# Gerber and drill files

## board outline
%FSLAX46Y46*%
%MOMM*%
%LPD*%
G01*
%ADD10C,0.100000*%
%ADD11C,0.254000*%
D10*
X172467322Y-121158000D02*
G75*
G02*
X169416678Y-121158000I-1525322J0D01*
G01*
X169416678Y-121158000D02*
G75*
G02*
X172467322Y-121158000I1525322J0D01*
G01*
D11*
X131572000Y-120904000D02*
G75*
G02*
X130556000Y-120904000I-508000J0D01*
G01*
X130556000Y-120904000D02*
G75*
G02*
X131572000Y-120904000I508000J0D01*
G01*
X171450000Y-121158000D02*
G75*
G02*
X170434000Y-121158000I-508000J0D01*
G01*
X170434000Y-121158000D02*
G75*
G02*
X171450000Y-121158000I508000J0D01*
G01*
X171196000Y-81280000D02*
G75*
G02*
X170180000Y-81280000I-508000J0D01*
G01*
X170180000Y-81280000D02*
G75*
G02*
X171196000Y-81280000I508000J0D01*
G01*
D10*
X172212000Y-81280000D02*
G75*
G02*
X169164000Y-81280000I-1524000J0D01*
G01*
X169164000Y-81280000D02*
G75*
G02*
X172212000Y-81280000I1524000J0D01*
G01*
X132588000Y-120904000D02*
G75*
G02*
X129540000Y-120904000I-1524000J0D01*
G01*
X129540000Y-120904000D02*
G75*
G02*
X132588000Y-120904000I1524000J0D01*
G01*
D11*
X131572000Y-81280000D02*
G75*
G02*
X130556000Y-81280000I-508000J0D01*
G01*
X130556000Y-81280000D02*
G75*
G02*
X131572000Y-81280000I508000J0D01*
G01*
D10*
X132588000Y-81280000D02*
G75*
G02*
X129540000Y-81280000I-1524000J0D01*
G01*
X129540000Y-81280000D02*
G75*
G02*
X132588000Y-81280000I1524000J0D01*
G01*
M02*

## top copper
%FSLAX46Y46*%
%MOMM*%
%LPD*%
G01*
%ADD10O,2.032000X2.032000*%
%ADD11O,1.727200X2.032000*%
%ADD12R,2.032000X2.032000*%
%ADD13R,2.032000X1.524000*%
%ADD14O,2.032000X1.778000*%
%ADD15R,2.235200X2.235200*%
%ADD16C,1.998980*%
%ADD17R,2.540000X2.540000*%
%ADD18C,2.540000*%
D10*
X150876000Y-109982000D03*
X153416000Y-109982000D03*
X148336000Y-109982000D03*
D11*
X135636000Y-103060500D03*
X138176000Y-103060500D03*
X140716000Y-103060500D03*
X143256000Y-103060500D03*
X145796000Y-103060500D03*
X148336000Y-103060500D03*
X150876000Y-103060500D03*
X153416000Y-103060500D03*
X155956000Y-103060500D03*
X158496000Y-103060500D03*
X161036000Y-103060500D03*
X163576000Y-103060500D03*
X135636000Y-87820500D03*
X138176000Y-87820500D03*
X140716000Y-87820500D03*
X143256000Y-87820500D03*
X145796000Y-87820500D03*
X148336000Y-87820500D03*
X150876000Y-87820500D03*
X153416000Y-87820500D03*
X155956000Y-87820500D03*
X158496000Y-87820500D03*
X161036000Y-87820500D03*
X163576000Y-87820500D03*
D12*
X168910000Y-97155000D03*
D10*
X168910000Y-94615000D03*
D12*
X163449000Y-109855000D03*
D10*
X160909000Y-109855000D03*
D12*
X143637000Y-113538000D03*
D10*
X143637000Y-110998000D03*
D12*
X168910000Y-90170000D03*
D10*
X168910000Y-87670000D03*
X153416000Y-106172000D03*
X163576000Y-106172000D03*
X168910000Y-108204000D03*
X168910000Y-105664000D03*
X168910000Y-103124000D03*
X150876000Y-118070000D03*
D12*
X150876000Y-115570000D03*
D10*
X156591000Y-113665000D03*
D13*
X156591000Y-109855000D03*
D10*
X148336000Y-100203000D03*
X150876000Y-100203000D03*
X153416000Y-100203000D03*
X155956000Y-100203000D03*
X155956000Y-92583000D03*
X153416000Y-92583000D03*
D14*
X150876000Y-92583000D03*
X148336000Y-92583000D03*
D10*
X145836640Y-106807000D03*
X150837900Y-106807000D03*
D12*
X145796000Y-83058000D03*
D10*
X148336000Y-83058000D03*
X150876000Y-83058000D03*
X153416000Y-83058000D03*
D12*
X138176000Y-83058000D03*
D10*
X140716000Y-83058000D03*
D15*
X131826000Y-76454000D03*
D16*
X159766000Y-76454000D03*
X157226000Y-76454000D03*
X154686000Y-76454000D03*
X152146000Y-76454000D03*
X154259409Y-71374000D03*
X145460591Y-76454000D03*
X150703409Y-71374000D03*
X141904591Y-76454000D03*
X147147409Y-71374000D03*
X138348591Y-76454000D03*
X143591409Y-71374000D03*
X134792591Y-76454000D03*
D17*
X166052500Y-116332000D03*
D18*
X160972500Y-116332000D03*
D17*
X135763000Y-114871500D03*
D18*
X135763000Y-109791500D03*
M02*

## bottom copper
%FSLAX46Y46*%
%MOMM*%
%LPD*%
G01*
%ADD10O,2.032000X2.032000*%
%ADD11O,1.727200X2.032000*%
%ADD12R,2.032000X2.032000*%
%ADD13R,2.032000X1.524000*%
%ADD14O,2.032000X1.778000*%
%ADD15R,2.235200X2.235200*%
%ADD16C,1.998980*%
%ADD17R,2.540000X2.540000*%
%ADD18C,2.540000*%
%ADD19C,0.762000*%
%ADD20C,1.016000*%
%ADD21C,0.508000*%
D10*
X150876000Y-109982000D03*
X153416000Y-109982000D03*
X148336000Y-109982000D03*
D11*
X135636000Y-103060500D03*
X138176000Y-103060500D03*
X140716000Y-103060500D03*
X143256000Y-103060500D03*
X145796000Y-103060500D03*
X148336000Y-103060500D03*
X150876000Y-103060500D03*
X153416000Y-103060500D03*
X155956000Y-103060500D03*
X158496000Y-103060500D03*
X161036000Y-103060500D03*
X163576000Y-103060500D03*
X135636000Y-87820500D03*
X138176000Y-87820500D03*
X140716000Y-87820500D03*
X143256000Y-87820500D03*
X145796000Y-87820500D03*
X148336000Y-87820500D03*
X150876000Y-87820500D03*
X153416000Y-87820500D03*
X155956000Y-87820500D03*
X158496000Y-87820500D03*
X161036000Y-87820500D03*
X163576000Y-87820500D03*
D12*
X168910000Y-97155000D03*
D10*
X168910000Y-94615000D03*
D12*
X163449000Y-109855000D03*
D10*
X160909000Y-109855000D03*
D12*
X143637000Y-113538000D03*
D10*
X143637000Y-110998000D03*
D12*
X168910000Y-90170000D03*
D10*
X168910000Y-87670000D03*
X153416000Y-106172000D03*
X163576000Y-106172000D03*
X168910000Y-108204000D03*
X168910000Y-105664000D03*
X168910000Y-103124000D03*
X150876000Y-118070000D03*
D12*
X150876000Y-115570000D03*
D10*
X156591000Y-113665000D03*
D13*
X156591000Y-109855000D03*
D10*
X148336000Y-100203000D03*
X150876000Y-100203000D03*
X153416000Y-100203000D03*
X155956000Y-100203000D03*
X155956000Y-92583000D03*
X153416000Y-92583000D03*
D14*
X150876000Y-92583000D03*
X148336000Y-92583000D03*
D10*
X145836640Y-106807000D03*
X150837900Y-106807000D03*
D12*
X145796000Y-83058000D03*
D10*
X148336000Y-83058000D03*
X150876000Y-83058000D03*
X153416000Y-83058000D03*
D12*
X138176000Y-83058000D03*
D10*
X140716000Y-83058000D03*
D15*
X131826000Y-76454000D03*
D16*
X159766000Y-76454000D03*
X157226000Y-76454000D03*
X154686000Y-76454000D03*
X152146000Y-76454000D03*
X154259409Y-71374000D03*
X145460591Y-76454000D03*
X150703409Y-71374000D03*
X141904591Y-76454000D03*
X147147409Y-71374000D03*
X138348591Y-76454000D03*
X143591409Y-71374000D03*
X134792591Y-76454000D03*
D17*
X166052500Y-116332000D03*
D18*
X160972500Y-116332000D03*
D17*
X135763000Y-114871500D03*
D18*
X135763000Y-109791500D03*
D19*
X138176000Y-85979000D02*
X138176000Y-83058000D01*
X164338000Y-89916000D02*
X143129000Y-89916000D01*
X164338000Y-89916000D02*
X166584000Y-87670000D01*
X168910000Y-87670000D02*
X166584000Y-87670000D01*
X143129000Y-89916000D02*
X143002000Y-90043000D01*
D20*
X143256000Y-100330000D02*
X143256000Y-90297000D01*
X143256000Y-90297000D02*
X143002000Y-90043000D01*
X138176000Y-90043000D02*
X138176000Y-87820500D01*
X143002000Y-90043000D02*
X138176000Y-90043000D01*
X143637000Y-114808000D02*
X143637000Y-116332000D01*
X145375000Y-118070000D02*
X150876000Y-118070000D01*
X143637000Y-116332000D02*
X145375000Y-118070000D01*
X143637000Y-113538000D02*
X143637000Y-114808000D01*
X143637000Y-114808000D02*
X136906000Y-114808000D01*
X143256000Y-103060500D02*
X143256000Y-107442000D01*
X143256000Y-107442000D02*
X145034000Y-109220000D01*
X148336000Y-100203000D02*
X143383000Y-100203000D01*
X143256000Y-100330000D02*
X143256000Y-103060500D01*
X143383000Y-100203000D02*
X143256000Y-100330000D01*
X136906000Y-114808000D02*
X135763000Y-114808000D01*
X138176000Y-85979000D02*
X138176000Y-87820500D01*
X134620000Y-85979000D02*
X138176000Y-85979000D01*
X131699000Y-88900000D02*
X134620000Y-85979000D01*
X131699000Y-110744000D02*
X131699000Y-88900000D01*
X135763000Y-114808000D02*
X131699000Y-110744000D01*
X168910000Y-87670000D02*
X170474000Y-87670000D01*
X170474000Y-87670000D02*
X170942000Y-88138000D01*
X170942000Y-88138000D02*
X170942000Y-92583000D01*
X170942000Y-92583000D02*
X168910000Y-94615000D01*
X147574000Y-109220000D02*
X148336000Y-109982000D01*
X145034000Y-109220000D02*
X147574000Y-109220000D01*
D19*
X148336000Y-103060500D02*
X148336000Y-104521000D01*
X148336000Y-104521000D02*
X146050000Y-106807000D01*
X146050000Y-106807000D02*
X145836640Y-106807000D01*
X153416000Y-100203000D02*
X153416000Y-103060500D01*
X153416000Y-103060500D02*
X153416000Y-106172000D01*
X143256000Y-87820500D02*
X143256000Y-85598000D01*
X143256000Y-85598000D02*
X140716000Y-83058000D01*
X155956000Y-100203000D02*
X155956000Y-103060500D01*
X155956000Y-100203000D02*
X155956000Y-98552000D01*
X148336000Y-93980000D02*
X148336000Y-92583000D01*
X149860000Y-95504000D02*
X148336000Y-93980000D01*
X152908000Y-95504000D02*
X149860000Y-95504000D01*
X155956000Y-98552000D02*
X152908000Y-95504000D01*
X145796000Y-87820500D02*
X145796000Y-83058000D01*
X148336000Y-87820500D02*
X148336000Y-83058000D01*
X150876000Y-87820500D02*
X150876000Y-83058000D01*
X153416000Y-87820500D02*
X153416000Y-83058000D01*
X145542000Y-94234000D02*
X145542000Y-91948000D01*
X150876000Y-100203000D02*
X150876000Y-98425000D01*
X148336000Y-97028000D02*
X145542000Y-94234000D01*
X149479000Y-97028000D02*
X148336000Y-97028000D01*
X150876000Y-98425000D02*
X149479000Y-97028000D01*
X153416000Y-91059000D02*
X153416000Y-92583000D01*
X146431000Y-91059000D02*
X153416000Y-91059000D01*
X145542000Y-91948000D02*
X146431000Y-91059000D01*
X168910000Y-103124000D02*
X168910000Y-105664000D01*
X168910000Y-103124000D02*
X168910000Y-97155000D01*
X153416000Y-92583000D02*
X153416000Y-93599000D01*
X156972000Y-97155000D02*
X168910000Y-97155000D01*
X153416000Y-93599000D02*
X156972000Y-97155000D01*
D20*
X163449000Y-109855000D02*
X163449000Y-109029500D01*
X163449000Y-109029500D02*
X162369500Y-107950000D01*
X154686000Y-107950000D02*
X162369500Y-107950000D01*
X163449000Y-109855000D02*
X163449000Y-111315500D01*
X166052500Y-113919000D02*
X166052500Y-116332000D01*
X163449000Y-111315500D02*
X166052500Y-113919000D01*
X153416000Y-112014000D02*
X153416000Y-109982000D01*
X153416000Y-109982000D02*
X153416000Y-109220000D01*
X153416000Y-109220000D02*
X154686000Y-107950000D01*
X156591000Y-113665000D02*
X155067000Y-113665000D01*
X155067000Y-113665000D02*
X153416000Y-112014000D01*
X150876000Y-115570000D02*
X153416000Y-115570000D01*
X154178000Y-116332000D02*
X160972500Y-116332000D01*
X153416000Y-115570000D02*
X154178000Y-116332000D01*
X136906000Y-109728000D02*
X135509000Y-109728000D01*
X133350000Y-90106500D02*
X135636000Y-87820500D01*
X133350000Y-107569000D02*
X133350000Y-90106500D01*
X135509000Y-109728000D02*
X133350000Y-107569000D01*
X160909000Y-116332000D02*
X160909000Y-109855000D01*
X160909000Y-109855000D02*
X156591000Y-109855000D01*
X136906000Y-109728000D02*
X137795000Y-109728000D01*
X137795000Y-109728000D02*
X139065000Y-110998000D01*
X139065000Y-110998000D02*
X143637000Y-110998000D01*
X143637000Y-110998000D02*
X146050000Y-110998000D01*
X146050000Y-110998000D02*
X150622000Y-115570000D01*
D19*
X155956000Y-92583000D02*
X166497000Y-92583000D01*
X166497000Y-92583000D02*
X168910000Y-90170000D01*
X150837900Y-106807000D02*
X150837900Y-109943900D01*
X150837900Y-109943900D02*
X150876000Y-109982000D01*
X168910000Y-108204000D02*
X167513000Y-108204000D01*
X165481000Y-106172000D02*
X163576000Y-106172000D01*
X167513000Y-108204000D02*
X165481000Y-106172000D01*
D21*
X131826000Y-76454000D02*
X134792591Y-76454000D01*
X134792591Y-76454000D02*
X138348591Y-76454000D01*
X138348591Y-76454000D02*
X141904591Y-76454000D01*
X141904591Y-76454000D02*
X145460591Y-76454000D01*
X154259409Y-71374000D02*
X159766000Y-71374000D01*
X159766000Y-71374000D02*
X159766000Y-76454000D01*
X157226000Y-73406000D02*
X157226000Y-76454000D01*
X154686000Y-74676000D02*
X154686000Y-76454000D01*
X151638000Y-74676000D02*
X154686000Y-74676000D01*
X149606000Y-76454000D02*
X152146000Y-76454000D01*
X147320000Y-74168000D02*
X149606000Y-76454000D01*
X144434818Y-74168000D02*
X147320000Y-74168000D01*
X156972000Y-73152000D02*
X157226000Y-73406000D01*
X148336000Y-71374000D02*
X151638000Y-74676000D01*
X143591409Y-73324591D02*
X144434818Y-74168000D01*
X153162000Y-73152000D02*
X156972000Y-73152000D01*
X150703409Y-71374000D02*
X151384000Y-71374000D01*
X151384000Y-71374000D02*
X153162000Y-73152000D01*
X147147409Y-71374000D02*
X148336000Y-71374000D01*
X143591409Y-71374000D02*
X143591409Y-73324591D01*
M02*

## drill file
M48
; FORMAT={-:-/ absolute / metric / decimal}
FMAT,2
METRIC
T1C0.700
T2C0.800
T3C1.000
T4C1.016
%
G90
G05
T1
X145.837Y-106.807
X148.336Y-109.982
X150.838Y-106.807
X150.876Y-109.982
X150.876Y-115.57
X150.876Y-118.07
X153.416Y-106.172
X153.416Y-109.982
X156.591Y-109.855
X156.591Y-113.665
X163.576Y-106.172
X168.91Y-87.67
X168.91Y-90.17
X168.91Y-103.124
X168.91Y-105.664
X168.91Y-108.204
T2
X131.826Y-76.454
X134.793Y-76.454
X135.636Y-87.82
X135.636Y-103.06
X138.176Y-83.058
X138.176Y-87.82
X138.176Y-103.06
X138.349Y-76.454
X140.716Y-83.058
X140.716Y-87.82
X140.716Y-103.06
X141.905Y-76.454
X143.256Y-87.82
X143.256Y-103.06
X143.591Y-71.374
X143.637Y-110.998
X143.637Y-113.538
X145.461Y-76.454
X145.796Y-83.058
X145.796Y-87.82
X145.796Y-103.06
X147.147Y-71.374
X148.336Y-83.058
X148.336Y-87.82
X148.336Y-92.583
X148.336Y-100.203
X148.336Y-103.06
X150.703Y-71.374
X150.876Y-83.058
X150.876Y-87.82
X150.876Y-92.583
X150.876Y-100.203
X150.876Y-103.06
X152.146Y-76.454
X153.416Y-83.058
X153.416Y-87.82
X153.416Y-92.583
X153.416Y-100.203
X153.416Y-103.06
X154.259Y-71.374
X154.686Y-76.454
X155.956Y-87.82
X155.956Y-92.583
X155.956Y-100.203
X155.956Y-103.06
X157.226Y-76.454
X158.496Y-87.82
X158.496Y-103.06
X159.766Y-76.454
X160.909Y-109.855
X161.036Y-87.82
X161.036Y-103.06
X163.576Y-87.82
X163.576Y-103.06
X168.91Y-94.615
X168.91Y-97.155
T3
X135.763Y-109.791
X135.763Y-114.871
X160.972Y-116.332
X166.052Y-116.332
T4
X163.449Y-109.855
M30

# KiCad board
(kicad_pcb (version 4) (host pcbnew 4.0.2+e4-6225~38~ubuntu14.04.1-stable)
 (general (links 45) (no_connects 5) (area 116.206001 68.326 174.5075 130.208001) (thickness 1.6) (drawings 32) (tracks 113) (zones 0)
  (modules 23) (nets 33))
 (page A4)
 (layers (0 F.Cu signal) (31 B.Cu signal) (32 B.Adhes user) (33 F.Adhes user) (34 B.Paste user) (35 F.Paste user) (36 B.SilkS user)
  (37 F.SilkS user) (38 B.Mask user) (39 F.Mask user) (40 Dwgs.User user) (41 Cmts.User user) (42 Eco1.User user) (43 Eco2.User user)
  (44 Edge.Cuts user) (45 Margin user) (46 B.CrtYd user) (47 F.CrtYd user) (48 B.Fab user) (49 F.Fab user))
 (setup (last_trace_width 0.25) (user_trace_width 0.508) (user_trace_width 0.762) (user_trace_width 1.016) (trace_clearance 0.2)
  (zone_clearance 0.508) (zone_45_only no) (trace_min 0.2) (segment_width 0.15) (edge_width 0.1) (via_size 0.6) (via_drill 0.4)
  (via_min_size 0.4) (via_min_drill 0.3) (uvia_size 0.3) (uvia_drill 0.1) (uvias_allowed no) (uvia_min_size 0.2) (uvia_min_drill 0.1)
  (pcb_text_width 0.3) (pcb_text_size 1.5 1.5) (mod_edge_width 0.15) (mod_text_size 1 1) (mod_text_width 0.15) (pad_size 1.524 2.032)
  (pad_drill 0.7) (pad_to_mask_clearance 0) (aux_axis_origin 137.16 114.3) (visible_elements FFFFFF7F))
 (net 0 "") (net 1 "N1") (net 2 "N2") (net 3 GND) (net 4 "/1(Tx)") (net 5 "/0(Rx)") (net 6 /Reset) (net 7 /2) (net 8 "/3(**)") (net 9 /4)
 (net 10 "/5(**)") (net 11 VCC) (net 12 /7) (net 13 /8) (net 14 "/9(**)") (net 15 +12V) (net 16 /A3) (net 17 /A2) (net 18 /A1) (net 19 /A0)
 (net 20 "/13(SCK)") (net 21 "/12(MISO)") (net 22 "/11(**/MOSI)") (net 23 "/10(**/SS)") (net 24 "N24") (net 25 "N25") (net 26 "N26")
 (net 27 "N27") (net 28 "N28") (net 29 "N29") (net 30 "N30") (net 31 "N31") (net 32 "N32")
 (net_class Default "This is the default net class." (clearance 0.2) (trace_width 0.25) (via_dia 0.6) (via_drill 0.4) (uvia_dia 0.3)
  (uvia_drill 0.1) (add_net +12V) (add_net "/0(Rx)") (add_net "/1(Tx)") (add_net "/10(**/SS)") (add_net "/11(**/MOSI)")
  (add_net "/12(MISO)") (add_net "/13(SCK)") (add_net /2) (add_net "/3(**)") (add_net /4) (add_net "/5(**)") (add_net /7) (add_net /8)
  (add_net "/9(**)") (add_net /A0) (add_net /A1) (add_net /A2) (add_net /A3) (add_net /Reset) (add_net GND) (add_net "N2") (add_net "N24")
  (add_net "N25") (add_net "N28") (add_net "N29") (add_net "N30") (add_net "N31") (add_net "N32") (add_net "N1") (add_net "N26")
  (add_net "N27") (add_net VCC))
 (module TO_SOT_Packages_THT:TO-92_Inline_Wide (layer F.Cu) (at 148.336 109.982)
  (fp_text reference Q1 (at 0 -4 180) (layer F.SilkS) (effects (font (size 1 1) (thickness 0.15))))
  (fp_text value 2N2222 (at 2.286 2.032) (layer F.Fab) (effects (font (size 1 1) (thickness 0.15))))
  (pad 2 thru_hole oval (at 2.54 0) (size 2.032 2.032) (drill 0.7) (layers *.Cu *.Mask F.SilkS) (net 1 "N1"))
  (pad 3 thru_hole oval (at 5.08 0) (size 2.032 2.032) (drill 0.7) (layers *.Cu *.Mask F.SilkS) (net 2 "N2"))
  (pad 1 thru_hole oval (at 0 0) (size 2.032 2.032) (drill 0.7) (layers *.Cu *.Mask F.SilkS) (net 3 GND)))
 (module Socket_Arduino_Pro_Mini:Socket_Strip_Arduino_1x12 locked (layer F.Cu) (at 135.636 103.0605)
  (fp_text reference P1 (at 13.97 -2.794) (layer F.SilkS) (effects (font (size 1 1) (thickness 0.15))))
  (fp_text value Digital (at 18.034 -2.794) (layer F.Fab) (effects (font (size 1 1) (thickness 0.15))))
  (pad 1 thru_hole oval (at 0 0) (size 1.7272 2.032) (drill 0.8) (layers *.Cu *.Mask F.SilkS) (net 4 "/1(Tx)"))
  (pad 2 thru_hole oval (at 2.54 0) (size 1.7272 2.032) (drill 0.8) (layers *.Cu *.Mask F.SilkS) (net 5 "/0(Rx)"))
  (pad 3 thru_hole oval (at 5.08 0) (size 1.7272 2.032) (drill 0.8) (layers *.Cu *.Mask F.SilkS) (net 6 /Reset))
  (pad 4 thru_hole oval (at 7.62 0) (size 1.7272 2.032) (drill 0.8) (layers *.Cu *.Mask F.SilkS) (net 3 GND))
  (pad 5 thru_hole oval (at 10.16 0) (size 1.7272 2.032) (drill 0.8) (layers *.Cu *.Mask F.SilkS) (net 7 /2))
  (pad 6 thru_hole oval (at 12.7 0) (size 1.7272 2.032) (drill 0.8) (layers *.Cu *.Mask F.SilkS) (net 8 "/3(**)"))
  (pad 7 thru_hole oval (at 15.24 0) (size 1.7272 2.032) (drill 0.8) (layers *.Cu *.Mask F.SilkS) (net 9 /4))
  (pad 8 thru_hole oval (at 17.78 0) (size 1.7272 2.032) (drill 0.8) (layers *.Cu *.Mask F.SilkS) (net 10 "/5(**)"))
  (pad 9 thru_hole oval (at 20.32 0) (size 1.7272 2.032) (drill 0.8) (layers *.Cu *.Mask F.SilkS) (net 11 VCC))
  (pad 10 thru_hole oval (at 22.86 0) (size 1.7272 2.032) (drill 0.8) (layers *.Cu *.Mask F.SilkS) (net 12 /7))
  (pad 11 thru_hole oval (at 25.4 0) (size 1.7272 2.032) (drill 0.8) (layers *.Cu *.Mask F.SilkS) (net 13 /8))
  (pad 12 thru_hole oval (at 27.94 0) (size 1.7272 2.032) (drill 0.8) (layers *.Cu *.Mask F.SilkS) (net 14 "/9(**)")))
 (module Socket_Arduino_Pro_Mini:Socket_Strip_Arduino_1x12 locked (layer F.Cu) (at 135.636 87.8205)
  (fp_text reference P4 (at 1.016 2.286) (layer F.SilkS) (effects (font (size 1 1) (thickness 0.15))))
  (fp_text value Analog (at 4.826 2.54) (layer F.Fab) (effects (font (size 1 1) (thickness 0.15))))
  (pad 1 thru_hole oval (at 0 0) (size 1.7272 2.032) (drill 0.8) (layers *.Cu *.Mask F.SilkS) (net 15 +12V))
  (pad 2 thru_hole oval (at 2.54 0) (size 1.7272 2.032) (drill 0.8) (layers *.Cu *.Mask F.SilkS) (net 3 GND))
  (pad 3 thru_hole oval (at 5.08 0) (size 1.7272 2.032) (drill 0.8) (layers *.Cu *.Mask F.SilkS) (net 6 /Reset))
  (pad 4 thru_hole oval (at 7.62 0) (size 1.7272 2.032) (drill 0.8) (layers *.Cu *.Mask F.SilkS) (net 11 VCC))
  (pad 5 thru_hole oval (at 10.16 0) (size 1.7272 2.032) (drill 0.8) (layers *.Cu *.Mask F.SilkS) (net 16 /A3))
  (pad 6 thru_hole oval (at 12.7 0) (size 1.7272 2.032) (drill 0.8) (layers *.Cu *.Mask F.SilkS) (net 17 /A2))
  (pad 7 thru_hole oval (at 15.24 0) (size 1.7272 2.032) (drill 0.8) (layers *.Cu *.Mask F.SilkS) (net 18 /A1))
  (pad 8 thru_hole oval (at 17.78 0) (size 1.7272 2.032) (drill 0.8) (layers *.Cu *.Mask F.SilkS) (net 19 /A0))
  (pad 9 thru_hole oval (at 20.32 0) (size 1.7272 2.032) (drill 0.8) (layers *.Cu *.Mask F.SilkS) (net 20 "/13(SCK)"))
  (pad 10 thru_hole oval (at 22.86 0) (size 1.7272 2.032) (drill 0.8) (layers *.Cu *.Mask F.SilkS) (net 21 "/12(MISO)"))
  (pad 11 thru_hole oval (at 25.4 0) (size 1.7272 2.032) (drill 0.8) (layers *.Cu *.Mask F.SilkS) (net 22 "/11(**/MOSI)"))
  (pad 12 thru_hole oval (at 27.94 0) (size 1.7272 2.032) (drill 0.8) (layers *.Cu *.Mask F.SilkS) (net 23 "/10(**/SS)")))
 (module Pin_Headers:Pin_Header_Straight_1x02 (layer F.Cu) (at 168.91 97.155 180)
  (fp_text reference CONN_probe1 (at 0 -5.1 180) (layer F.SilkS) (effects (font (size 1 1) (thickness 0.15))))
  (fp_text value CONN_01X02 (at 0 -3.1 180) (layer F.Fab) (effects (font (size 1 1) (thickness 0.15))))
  (pad 1 thru_hole rect (at 0 0 180) (size 2.032 2.032) (drill 0.8) (layers *.Cu *.Mask F.SilkS) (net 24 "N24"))
  (pad 2 thru_hole oval (at 0 2.54 180) (size 2.032 2.032) (drill 0.8) (layers *.Cu *.Mask F.SilkS) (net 3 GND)))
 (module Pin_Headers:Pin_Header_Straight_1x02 (layer F.Cu) (at 163.449 109.855 270)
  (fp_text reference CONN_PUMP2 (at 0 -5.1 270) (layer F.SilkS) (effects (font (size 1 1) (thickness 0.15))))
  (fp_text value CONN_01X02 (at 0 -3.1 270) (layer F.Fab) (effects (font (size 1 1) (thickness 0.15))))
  (pad 1 thru_hole rect (at 0 0 270) (size 2.032 2.032) (drill 1.016) (layers *.Cu *.Mask F.SilkS) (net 2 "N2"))
  (pad 2 thru_hole oval (at 0 2.54 270) (size 2.032 2.032) (drill 0.8) (layers *.Cu *.Mask F.SilkS) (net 15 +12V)))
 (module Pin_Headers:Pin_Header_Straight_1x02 (layer F.Cu) (at 143.637 113.538 180)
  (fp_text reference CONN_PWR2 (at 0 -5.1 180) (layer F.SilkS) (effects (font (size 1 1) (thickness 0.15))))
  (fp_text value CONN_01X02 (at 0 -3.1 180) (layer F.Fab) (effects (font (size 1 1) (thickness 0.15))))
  (pad 1 thru_hole rect (at 0 0 180) (size 2.032 2.032) (drill 0.8) (layers *.Cu *.Mask F.SilkS) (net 3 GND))
  (pad 2 thru_hole oval (at 0 2.54 180) (size 2.032 2.032) (drill 0.8) (layers *.Cu *.Mask F.SilkS) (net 15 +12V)))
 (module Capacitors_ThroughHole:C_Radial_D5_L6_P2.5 (layer F.Cu) (at 168.91 90.17 90)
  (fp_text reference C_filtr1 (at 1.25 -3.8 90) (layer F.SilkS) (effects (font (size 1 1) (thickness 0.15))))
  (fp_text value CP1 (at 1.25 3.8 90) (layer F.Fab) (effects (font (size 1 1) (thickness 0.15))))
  (pad 1 thru_hole rect (at 0 0 90) (size 2.032 2.032) (drill 0.7) (layers *.Cu *.Mask F.SilkS) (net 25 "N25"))
  (pad 2 thru_hole oval (at 2.5 0 90) (size 2.032 2.032) (drill 0.7) (layers *.Cu *.Mask F.SilkS) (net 3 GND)))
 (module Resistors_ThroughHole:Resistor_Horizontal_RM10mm (layer F.Cu) (at 158.496 106.172)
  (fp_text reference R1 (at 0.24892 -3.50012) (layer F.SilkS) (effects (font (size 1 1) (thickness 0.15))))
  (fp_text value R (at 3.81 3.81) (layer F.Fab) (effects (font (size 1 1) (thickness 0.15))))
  (pad 1 thru_hole oval (at -5.08 0) (size 2.032 2.032) (drill 0.7) (layers *.Cu *.Mask F.SilkS) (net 10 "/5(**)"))
  (pad 2 thru_hole oval (at 5.08 0) (size 2.032 2.032) (drill 0.7) (layers *.Cu *.Mask F.SilkS) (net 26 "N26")))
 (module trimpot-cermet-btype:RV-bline (layer F.Cu) (at 168.91 105.664 90)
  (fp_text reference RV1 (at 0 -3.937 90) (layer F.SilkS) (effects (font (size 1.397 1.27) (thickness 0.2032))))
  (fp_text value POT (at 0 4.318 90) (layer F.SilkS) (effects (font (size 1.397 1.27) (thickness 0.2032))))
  (pad 1 thru_hole oval (at -2.54 0 90) (size 2.032 2.032) (drill 0.7) (layers *.Cu *.Mask F.SilkS) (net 26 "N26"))
  (pad 2 thru_hole oval (at 0 0 90) (size 2.032 2.032) (drill 0.7) (layers *.Cu *.Mask F.SilkS) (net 24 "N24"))
  (pad 3 thru_hole oval (at 2.54 0 90) (size 2.032 2.032) (drill 0.7) (layers *.Cu *.Mask F.SilkS) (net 24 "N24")))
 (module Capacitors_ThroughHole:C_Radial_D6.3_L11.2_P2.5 (layer F.Cu) (at 150.876 115.57 270)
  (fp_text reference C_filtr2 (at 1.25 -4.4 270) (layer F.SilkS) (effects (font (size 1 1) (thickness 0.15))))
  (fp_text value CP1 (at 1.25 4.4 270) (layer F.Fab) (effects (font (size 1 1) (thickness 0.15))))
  (pad 2 thru_hole oval (at 2.5 0 270) (size 2.032 2.032) (drill 0.7) (layers *.Cu *.Mask F.SilkS) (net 3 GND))
  (pad 1 thru_hole rect (at 0 0 270) (size 2.032 2.032) (drill 0.7) (layers *.Cu *.Mask F.SilkS) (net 15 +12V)))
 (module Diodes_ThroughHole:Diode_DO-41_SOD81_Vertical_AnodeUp (layer F.Cu) (at 156.591 109.855 270)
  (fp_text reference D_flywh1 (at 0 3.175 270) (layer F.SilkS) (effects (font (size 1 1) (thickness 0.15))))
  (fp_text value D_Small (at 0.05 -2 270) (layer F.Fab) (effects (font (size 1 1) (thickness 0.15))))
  (pad 2 thru_hole oval (at 3.81 0 270) (size 2.032 2.032) (drill 0.7) (layers *.Cu *.Mask F.SilkS) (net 2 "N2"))
  (pad 1 thru_hole rect (at 0 0 270) (size 1.524 2.032) (drill 0.7) (layers *.Cu *.Mask F.SilkS) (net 15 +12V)))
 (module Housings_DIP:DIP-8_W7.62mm (layer F.Cu) (at 148.336 100.203 90)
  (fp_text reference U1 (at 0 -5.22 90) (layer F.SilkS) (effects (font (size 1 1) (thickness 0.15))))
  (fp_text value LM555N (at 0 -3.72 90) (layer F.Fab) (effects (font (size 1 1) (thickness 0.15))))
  (pad 1 thru_hole oval (at 0 0 90) (size 2.032 2.032) (drill 0.8) (layers *.Cu *.Mask F.SilkS) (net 3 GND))
  (pad 2 thru_hole oval (at 0 2.54 90) (size 2.032 2.032) (drill 0.8) (layers *.Cu *.Mask F.SilkS) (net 24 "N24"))
  (pad 3 thru_hole oval (at 0 5.08 90) (size 2.032 2.032) (drill 0.8) (layers *.Cu *.Mask F.SilkS) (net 10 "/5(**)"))
  (pad 4 thru_hole oval (at 0 7.62 90) (size 2.032 2.032) (drill 0.8) (layers *.Cu *.Mask F.SilkS) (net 11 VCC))
  (pad 5 thru_hole oval (at 7.62 7.62 90) (size 2.032 2.032) (drill 0.8) (layers *.Cu *.Mask F.SilkS) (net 25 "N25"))
  (pad 6 thru_hole oval (at 7.62 5.08 90) (size 2.032 2.032) (drill 0.8) (layers *.Cu *.Mask F.SilkS) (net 24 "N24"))
  (pad 7 thru_hole oval (at 7.62 2.54 90) (size 1.778 2.032) (drill 0.8) (layers *.Cu *.Mask F.SilkS) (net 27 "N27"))
  (pad 8 thru_hole oval (at 7.62 0 90) (size 1.778 2.032) (drill 0.8) (layers *.Cu *.Mask F.SilkS) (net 11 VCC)))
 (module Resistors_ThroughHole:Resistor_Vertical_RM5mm (layer F.Cu) (at 148.336 106.807)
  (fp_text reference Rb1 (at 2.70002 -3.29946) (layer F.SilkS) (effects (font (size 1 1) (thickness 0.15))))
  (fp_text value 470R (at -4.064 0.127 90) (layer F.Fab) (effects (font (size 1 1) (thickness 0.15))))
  (pad 1 thru_hole oval (at -2.49936 0) (size 2.032 2.032) (drill 0.7) (layers *.Cu *.Mask F.SilkS) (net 8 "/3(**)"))
  (pad 2 thru_hole oval (at 2.5019 0) (size 2.032 2.032) (drill 0.7) (layers *.Cu *.Mask F.SilkS) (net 1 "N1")))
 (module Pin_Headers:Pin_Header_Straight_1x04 (layer F.Cu) (at 145.796 83.058 90)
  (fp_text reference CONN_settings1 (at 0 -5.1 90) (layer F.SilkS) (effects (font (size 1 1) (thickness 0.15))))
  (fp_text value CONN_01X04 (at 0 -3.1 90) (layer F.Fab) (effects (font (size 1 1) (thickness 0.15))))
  (pad 1 thru_hole rect (at 0 0 90) (size 2.032 2.032) (drill 0.8) (layers *.Cu *.Mask F.SilkS) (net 16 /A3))
  (pad 2 thru_hole oval (at 0 2.54 90) (size 2.032 2.032) (drill 0.8) (layers *.Cu *.Mask F.SilkS) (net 17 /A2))
  (pad 3 thru_hole oval (at 0 5.08 90) (size 2.032 2.032) (drill 0.8) (layers *.Cu *.Mask F.SilkS) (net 18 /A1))
  (pad 4 thru_hole oval (at 0 7.62 90) (size 2.032 2.032) (drill 0.8) (layers *.Cu *.Mask F.SilkS) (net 19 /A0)))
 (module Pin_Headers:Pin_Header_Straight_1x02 (layer F.Cu) (at 138.176 83.058 90)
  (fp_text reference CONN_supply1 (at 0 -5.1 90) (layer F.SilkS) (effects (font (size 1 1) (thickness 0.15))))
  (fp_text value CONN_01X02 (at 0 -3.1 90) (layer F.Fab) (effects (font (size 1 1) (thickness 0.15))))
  (pad 1 thru_hole rect (at 0 0 90) (size 2.032 2.032) (drill 0.8) (layers *.Cu *.Mask F.SilkS) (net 3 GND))
  (pad 2 thru_hole oval (at 0 2.54 90) (size 2.032 2.032) (drill 0.8) (layers *.Cu *.Mask F.SilkS) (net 11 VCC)))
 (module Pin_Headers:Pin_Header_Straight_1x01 (layer F.Cu) (at 131.826 76.454)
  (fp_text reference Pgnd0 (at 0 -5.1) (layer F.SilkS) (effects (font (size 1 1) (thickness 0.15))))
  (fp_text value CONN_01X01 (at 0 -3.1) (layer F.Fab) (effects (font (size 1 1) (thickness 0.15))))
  (pad 1 thru_hole rect (at 0 0) (size 2.2352 2.2352) (drill 0.8) (layers *.Cu *.Mask F.SilkS) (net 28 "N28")))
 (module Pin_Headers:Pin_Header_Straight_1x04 (layer F.Cu) (at 159.766 76.454 270)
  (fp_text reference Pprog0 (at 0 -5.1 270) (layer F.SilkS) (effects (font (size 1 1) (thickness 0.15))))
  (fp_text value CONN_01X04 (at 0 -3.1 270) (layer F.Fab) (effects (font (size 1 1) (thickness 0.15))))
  (pad 1 thru_hole circle (at 0 0 270) (size 1.99898 1.99898) (drill 0.8) (layers *.Cu *.SilkS *.Mask) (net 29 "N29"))
  (pad 2 thru_hole circle (at 0 2.54 270) (size 1.99898 1.99898) (drill 0.8) (layers *.Cu *.SilkS *.Mask) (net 29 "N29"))
  (pad 3 thru_hole circle (at 0 5.08 270) (size 1.99898 1.99898) (drill 0.8) (layers *.Cu *.SilkS *.Mask) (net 29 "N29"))
  (pad 4 thru_hole circle (at 0 7.62 270) (size 1.99898 1.99898) (drill 0.8) (layers *.Cu *.SilkS *.Mask) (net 29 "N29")))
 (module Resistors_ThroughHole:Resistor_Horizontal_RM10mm (layer F.Cu) (at 149.86 73.914 210)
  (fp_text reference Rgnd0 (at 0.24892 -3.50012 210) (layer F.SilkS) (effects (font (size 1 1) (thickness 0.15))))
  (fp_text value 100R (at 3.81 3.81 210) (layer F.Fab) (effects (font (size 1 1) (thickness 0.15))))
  (pad 1 thru_hole circle (at -5.08 0 210) (size 1.99898 1.99898) (drill 0.8) (layers *.Cu *.SilkS *.Mask) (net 29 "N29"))
  (pad 2 thru_hole circle (at 5.08 0 210) (size 1.99898 1.99898) (drill 0.8) (layers *.Cu *.SilkS *.Mask) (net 28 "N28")))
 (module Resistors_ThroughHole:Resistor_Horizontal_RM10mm (layer F.Cu) (at 146.304 73.914 210)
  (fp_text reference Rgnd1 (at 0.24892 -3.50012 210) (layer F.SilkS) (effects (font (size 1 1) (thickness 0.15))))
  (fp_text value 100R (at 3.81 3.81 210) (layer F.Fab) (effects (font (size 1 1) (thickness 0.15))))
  (pad 1 thru_hole circle (at -5.08 0 210) (size 1.99898 1.99898) (drill 0.8) (layers *.Cu *.SilkS *.Mask) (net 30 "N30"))
  (pad 2 thru_hole circle (at 5.08 0 210) (size 1.99898 1.99898) (drill 0.8) (layers *.Cu *.SilkS *.Mask) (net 28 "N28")))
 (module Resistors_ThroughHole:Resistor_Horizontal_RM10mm (layer F.Cu) (at 142.748 73.914 210)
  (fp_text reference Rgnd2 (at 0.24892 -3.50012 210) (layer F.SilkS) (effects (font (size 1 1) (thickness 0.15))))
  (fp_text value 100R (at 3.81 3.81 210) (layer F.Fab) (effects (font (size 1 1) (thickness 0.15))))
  (pad 1 thru_hole circle (at -5.08 0 210) (size 1.99898 1.99898) (drill 0.8) (layers *.Cu *.SilkS *.Mask) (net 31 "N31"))
  (pad 2 thru_hole circle (at 5.08 0 210) (size 1.99898 1.99898) (drill 0.8) (layers *.Cu *.SilkS *.Mask) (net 28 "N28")))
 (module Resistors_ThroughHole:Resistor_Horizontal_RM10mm (layer F.Cu) (at 139.192 73.914 210)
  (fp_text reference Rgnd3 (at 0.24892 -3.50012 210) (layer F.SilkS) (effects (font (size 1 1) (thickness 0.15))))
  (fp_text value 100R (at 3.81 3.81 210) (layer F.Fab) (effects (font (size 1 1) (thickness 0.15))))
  (pad 1 thru_hole circle (at -5.08 0 210) (size 1.99898 1.99898) (drill 0.8) (layers *.Cu *.SilkS *.Mask) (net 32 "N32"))
  (pad 2 thru_hole circle (at 5.08 0 210) (size 1.99898 1.99898) (drill 0.8) (layers *.Cu *.SilkS *.Mask) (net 28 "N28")))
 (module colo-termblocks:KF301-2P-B (layer F.Cu) (at 163.5125 116.332)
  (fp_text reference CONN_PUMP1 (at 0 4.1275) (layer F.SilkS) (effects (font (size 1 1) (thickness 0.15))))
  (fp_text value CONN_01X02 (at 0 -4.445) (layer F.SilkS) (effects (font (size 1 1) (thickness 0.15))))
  (pad 1 thru_hole rect (at 2.54 0) (size 2.54 2.54) (drill 1) (layers *.Cu *.Mask F.SilkS) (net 2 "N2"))
  (pad 2 thru_hole circle (at -2.54 0) (size 2.54 2.54) (drill 1) (layers *.Cu *.Mask F.SilkS) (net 15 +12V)))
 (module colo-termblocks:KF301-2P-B (layer F.Cu) (at 135.763 112.3315 270)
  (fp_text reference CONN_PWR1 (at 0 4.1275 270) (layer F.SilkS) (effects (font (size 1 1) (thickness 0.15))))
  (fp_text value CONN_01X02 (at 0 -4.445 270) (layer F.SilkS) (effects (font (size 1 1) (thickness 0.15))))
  (pad 1 thru_hole rect (at 2.54 0 270) (size 2.54 2.54) (drill 1) (layers *.Cu *.Mask F.SilkS) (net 3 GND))
  (pad 2 thru_hole circle (at -2.54 0 270) (size 2.54 2.54) (drill 1) (layers *.Cu *.Mask F.SilkS) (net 15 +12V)))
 (gr_circle (center 170.942 121.158) (end 172.466 121.2215) (layer Edge.Cuts) (width 0.1))
 (gr_circle (center 131.064 120.904) (end 130.556 120.904) (layer Edge.Cuts) (width 0.254))
 (gr_circle (center 170.942 121.158) (end 170.434 121.158) (layer Edge.Cuts) (width 0.254))
 (gr_circle (center 170.688 81.28) (end 170.18 81.28) (layer Edge.Cuts) (width 0.254))
 (gr_circle (center 170.688 81.28) (end 169.164 81.28) (layer Edge.Cuts) (width 0.1))
 (gr_circle (center 131.064 120.904) (end 129.54 120.904) (layer Edge.Cuts) (width 0.1))
 (gr_circle (center 131.064 81.28) (end 130.556 81.28) (layer Edge.Cuts) (width 0.254))
 (gr_circle (center 131.064 81.28) (end 129.54 81.28) (layer Edge.Cuts) (width 0.1))
 (segment (start 138.176 85.979) (end 138.176 83.058) (width 0.762) (layer B.Cu) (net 3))
 (segment (start 164.338 89.916) (end 143.129 89.916) (width 0.762) (layer B.Cu) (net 3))
 (segment (start 164.338 89.916) (end 166.584 87.67) (width 0.762) (layer B.Cu) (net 3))
 (segment (start 168.91 87.67) (end 166.584 87.67) (width 0.762) (layer B.Cu) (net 3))
 (segment (start 143.129 89.916) (end 143.002 90.043) (width 0.762) (layer B.Cu) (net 3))
 (segment (start 143.256 100.33) (end 143.256 90.297) (width 1.016) (layer B.Cu) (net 3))
 (segment (start 143.256 90.297) (end 143.002 90.043) (width 1.016) (layer B.Cu) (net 3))
 (segment (start 138.176 90.043) (end 138.176 87.8205) (width 1.016) (layer B.Cu) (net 3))
 (segment (start 143.002 90.043) (end 138.176 90.043) (width 1.016) (layer B.Cu) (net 3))
 (segment (start 143.637 114.808) (end 143.637 116.332) (width 1.016) (layer B.Cu) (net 3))
 (segment (start 145.375 118.07) (end 150.876 118.07) (width 1.016) (layer B.Cu) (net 3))
 (segment (start 143.637 116.332) (end 145.375 118.07) (width 1.016) (layer B.Cu) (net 3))
 (segment (start 143.637 113.538) (end 143.637 114.808) (width 1.016) (layer B.Cu) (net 3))
 (segment (start 143.637 114.808) (end 136.906 114.808) (width 1.016) (layer B.Cu) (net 3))
 (segment (start 143.256 103.0605) (end 143.256 107.442) (width 1.016) (layer B.Cu) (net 3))
 (segment (start 143.256 107.442) (end 145.034 109.22) (width 1.016) (layer B.Cu) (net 3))
 (segment (start 148.336 100.203) (end 143.383 100.203) (width 1.016) (layer B.Cu) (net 3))
 (segment (start 143.256 100.33) (end 143.256 103.0605) (width 1.016) (layer B.Cu) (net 3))
 (segment (start 143.383 100.203) (end 143.256 100.33) (width 1.016) (layer B.Cu) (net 3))
 (segment (start 136.906 114.808) (end 135.763 114.808) (width 1.016) (layer B.Cu) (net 3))
 (segment (start 138.176 85.979) (end 138.176 87.8205) (width 1.016) (layer B.Cu) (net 3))
 (segment (start 134.62 85.979) (end 138.176 85.979) (width 1.016) (layer B.Cu) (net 3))
 (segment (start 131.699 88.9) (end 134.62 85.979) (width 1.016) (layer B.Cu) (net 3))
 (segment (start 131.699 110.744) (end 131.699 88.9) (width 1.016) (layer B.Cu) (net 3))
 (segment (start 135.763 114.808) (end 131.699 110.744) (width 1.016) (layer B.Cu) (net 3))
 (segment (start 168.91 87.67) (end 170.474 87.67) (width 1.016) (layer B.Cu) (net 3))
 (segment (start 170.474 87.67) (end 170.942 88.138) (width 1.016) (layer B.Cu) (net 3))
 (segment (start 170.942 88.138) (end 170.942 92.583) (width 1.016) (layer B.Cu) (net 3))
 (segment (start 170.942 92.583) (end 168.91 94.615) (width 1.016) (layer B.Cu) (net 3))
 (segment (start 147.574 109.22) (end 148.336 109.982) (width 1.016) (layer B.Cu) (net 3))
 (segment (start 145.034 109.22) (end 147.574 109.22) (width 1.016) (layer B.Cu) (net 3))
 (segment (start 148.336 103.0605) (end 148.336 104.521) (width 0.762) (layer B.Cu) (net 8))
 (segment (start 148.336 104.521) (end 146.05 106.807) (width 0.762) (layer B.Cu) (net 8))
 (segment (start 146.05 106.807) (end 145.83664 106.807) (width 0.762) (layer B.Cu) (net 8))
 (segment (start 153.416 100.203) (end 153.416 103.0605) (width 0.762) (layer B.Cu) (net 10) (status 10))
 (segment (start 153.416 103.0605) (end 153.416 106.172) (width 0.762) (layer B.Cu) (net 10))
 (segment (start 143.256 87.8205) (end 143.256 85.598) (width 0.762) (layer B.Cu) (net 11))
 (segment (start 143.256 85.598) (end 140.716 83.058) (width 0.762) (layer B.Cu) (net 11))
 (segment (start 155.956 100.203) (end 155.956 103.0605) (width 0.762) (layer B.Cu) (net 11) (status 10))
 (segment (start 155.956 100.203) (end 155.956 98.552) (width 0.762) (layer B.Cu) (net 11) (status 10))
 (segment (start 148.336 93.98) (end 148.336 92.583) (width 0.762) (layer B.Cu) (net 11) (status 20))
 (segment (start 149.86 95.504) (end 148.336 93.98) (width 0.762) (layer B.Cu) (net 11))
 (segment (start 152.908 95.504) (end 149.86 95.504) (width 0.762) (layer B.Cu) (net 11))
 (segment (start 155.956 98.552) (end 152.908 95.504) (width 0.762) (layer B.Cu) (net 11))
 (segment (start 145.796 87.8205) (end 145.796 83.058) (width 0.762) (layer B.Cu) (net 16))
 (segment (start 148.336 87.8205) (end 148.336 83.058) (width 0.762) (layer B.Cu) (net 17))
 (segment (start 150.876 87.8205) (end 150.876 83.058) (width 0.762) (layer B.Cu) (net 18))
 (segment (start 153.416 87.8205) (end 153.416 83.058) (width 0.762) (layer B.Cu) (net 19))
 (segment (start 145.542 94.234) (end 145.542 91.948) (width 0.762) (layer B.Cu) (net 24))
 (segment (start 150.876 100.203) (end 150.876 98.425) (width 0.762) (layer B.Cu) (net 24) (status 10))
 (segment (start 148.336 97.028) (end 145.542 94.234) (width 0.762) (layer B.Cu) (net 24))
 (segment (start 149.479 97.028) (end 148.336 97.028) (width 0.762) (layer B.Cu) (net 24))
 (segment (start 150.876 98.425) (end 149.479 97.028) (width 0.762) (layer B.Cu) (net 24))
 (segment (start 153.416 91.059) (end 153.416 92.583) (width 0.762) (layer B.Cu) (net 24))
 (segment (start 146.431 91.059) (end 153.416 91.059) (width 0.762) (layer B.Cu) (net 24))
 (segment (start 145.542 91.948) (end 146.431 91.059) (width 0.762) (layer B.Cu) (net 24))
 (segment (start 168.91 103.124) (end 168.91 105.664) (width 0.762) (layer B.Cu) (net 24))
 (segment (start 168.91 103.124) (end 168.91 97.155) (width 0.762) (layer B.Cu) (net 24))
 (segment (start 153.416 92.583) (end 153.416 93.599) (width 0.762) (layer B.Cu) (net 24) (status 10))
 (segment (start 156.972 97.155) (end 168.91 97.155) (width 0.762) (layer B.Cu) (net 24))
 (segment (start 153.416 93.599) (end 156.972 97.155) (width 0.762) (layer B.Cu) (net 24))
 (segment (start 163.449 109.855) (end 163.449 109.0295) (width 1.016) (layer B.Cu) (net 2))
 (segment (start 163.449 109.0295) (end 162.3695 107.95) (width 1.016) (layer B.Cu) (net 2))
 (segment (start 154.686 107.95) (end 162.3695 107.95) (width 1.016) (layer B.Cu) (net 2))
 (segment (start 163.449 109.855) (end 163.449 111.3155) (width 1.016) (layer B.Cu) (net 2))
 (segment (start 166.0525 113.919) (end 166.0525 116.332) (width 1.016) (layer B.Cu) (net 2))
 (segment (start 163.449 111.3155) (end 166.0525 113.919) (width 1.016) (layer B.Cu) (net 2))
 (segment (start 153.416 112.014) (end 153.416 109.982) (width 1.016) (layer B.Cu) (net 2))
 (segment (start 153.416 109.982) (end 153.416 109.22) (width 1.016) (layer B.Cu) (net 2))
 (segment (start 153.416 109.22) (end 154.686 107.95) (width 1.016) (layer B.Cu) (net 2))
 (segment (start 156.591 113.665) (end 155.067 113.665) (width 1.016) (layer B.Cu) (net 2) (status 10))
 (segment (start 155.067 113.665) (end 153.416 112.014) (width 1.016) (layer B.Cu) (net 2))
 (segment (start 150.876 115.57) (end 153.416 115.57) (width 1.016) (layer B.Cu) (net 15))
 (segment (start 154.178 116.332) (end 160.9725 116.332) (width 1.016) (layer B.Cu) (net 15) (status 20))
 (segment (start 153.416 115.57) (end 154.178 116.332) (width 1.016) (layer B.Cu) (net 15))
 (segment (start 136.906 109.728) (end 135.509 109.728) (width 1.016) (layer B.Cu) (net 15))
 (segment (start 133.35 90.1065) (end 135.636 87.8205) (width 1.016) (layer B.Cu) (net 15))
 (segment (start 133.35 107.569) (end 133.35 90.1065) (width 1.016) (layer B.Cu) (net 15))
 (segment (start 135.509 109.728) (end 133.35 107.569) (width 1.016) (layer B.Cu) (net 15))
 (segment (start 160.909 116.332) (end 160.909 109.855) (width 1.016) (layer B.Cu) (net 15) (status 10))
 (segment (start 160.909 109.855) (end 156.591 109.855) (width 1.016) (layer B.Cu) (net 15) (status 10))
 (segment (start 136.906 109.728) (end 137.795 109.728) (width 1.016) (layer B.Cu) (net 15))
 (segment (start 137.795 109.728) (end 139.065 110.998) (width 1.016) (layer B.Cu) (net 15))
 (segment (start 139.065 110.998) (end 143.637 110.998) (width 1.016) (layer B.Cu) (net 15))
 (segment (start 143.637 110.998) (end 146.05 110.998) (width 1.016) (layer B.Cu) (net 15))
 (segment (start 146.05 110.998) (end 150.622 115.57) (width 1.016) (layer B.Cu) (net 15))
 (segment (start 155.956 92.583) (end 166.497 92.583) (width 0.762) (layer B.Cu) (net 25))
 (segment (start 166.497 92.583) (end 168.91 90.17) (width 0.762) (layer B.Cu) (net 25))
 (segment (start 150.8379 106.807) (end 150.8379 109.9439) (width 0.762) (layer B.Cu) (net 1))
 (segment (start 150.8379 109.9439) (end 150.876 109.982) (width 0.762) (layer B.Cu) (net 1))
 (segment (start 168.91 108.204) (end 167.513 108.204) (width 0.762) (layer B.Cu) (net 26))
 (segment (start 165.481 106.172) (end 163.576 106.172) (width 0.762) (layer B.Cu) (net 26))
 (segment (start 167.513 108.204) (end 165.481 106.172) (width 0.762) (layer B.Cu) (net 26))
 (segment (start 131.826 76.454) (end 134.792591 76.454) (width 0.508) (layer B.Cu) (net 28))
 (segment (start 134.792591 76.454) (end 138.348591 76.454) (width 0.508) (layer B.Cu) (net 28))
 (segment (start 138.348591 76.454) (end 141.904591 76.454) (width 0.508) (layer B.Cu) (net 28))
 (segment (start 141.904591 76.454) (end 145.460591 76.454) (width 0.508) (layer B.Cu) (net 28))
 (segment (start 154.259409 71.374) (end 159.766 71.374) (width 0.508) (layer B.Cu) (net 29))
 (segment (start 159.766 71.374) (end 159.766 76.454) (width 0.508) (layer B.Cu) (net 29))
 (segment (start 157.226 73.406) (end 157.226 76.454) (width 0.508) (layer B.Cu) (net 29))
 (segment (start 154.686 74.676) (end 154.686 76.454) (width 0.508) (layer B.Cu) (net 29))
 (segment (start 151.638 74.676) (end 154.686 74.676) (width 0.508) (layer B.Cu) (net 29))
 (segment (start 149.606 76.454) (end 152.146 76.454) (width 0.508) (layer B.Cu) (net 29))
 (segment (start 147.32 74.168) (end 149.606 76.454) (width 0.508) (layer B.Cu) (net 29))
 (segment (start 144.434818 74.168) (end 147.32 74.168) (width 0.508) (layer B.Cu) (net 29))
 (segment (start 156.972 73.152) (end 157.226 73.406) (width 0.508) (layer B.Cu) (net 29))
 (segment (start 148.336 71.374) (end 151.638 74.676) (width 0.508) (layer B.Cu) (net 29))
 (segment (start 143.591409 73.324591) (end 144.434818 74.168) (width 0.508) (layer B.Cu) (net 29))
 (segment (start 153.162 73.152) (end 156.972 73.152) (width 0.508) (layer B.Cu) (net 29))
 (segment (start 150.703409 71.374) (end 151.384 71.374) (width 0.508) (layer B.Cu) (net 30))
 (segment (start 151.384 71.374) (end 153.162 73.152) (width 0.508) (layer B.Cu) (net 30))
 (segment (start 147.147409 71.374) (end 148.336 71.374) (width 0.508) (layer B.Cu) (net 31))
 (segment (start 143.591409 71.374) (end 143.591409 73.324591) (width 0.508) (layer B.Cu) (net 32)))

